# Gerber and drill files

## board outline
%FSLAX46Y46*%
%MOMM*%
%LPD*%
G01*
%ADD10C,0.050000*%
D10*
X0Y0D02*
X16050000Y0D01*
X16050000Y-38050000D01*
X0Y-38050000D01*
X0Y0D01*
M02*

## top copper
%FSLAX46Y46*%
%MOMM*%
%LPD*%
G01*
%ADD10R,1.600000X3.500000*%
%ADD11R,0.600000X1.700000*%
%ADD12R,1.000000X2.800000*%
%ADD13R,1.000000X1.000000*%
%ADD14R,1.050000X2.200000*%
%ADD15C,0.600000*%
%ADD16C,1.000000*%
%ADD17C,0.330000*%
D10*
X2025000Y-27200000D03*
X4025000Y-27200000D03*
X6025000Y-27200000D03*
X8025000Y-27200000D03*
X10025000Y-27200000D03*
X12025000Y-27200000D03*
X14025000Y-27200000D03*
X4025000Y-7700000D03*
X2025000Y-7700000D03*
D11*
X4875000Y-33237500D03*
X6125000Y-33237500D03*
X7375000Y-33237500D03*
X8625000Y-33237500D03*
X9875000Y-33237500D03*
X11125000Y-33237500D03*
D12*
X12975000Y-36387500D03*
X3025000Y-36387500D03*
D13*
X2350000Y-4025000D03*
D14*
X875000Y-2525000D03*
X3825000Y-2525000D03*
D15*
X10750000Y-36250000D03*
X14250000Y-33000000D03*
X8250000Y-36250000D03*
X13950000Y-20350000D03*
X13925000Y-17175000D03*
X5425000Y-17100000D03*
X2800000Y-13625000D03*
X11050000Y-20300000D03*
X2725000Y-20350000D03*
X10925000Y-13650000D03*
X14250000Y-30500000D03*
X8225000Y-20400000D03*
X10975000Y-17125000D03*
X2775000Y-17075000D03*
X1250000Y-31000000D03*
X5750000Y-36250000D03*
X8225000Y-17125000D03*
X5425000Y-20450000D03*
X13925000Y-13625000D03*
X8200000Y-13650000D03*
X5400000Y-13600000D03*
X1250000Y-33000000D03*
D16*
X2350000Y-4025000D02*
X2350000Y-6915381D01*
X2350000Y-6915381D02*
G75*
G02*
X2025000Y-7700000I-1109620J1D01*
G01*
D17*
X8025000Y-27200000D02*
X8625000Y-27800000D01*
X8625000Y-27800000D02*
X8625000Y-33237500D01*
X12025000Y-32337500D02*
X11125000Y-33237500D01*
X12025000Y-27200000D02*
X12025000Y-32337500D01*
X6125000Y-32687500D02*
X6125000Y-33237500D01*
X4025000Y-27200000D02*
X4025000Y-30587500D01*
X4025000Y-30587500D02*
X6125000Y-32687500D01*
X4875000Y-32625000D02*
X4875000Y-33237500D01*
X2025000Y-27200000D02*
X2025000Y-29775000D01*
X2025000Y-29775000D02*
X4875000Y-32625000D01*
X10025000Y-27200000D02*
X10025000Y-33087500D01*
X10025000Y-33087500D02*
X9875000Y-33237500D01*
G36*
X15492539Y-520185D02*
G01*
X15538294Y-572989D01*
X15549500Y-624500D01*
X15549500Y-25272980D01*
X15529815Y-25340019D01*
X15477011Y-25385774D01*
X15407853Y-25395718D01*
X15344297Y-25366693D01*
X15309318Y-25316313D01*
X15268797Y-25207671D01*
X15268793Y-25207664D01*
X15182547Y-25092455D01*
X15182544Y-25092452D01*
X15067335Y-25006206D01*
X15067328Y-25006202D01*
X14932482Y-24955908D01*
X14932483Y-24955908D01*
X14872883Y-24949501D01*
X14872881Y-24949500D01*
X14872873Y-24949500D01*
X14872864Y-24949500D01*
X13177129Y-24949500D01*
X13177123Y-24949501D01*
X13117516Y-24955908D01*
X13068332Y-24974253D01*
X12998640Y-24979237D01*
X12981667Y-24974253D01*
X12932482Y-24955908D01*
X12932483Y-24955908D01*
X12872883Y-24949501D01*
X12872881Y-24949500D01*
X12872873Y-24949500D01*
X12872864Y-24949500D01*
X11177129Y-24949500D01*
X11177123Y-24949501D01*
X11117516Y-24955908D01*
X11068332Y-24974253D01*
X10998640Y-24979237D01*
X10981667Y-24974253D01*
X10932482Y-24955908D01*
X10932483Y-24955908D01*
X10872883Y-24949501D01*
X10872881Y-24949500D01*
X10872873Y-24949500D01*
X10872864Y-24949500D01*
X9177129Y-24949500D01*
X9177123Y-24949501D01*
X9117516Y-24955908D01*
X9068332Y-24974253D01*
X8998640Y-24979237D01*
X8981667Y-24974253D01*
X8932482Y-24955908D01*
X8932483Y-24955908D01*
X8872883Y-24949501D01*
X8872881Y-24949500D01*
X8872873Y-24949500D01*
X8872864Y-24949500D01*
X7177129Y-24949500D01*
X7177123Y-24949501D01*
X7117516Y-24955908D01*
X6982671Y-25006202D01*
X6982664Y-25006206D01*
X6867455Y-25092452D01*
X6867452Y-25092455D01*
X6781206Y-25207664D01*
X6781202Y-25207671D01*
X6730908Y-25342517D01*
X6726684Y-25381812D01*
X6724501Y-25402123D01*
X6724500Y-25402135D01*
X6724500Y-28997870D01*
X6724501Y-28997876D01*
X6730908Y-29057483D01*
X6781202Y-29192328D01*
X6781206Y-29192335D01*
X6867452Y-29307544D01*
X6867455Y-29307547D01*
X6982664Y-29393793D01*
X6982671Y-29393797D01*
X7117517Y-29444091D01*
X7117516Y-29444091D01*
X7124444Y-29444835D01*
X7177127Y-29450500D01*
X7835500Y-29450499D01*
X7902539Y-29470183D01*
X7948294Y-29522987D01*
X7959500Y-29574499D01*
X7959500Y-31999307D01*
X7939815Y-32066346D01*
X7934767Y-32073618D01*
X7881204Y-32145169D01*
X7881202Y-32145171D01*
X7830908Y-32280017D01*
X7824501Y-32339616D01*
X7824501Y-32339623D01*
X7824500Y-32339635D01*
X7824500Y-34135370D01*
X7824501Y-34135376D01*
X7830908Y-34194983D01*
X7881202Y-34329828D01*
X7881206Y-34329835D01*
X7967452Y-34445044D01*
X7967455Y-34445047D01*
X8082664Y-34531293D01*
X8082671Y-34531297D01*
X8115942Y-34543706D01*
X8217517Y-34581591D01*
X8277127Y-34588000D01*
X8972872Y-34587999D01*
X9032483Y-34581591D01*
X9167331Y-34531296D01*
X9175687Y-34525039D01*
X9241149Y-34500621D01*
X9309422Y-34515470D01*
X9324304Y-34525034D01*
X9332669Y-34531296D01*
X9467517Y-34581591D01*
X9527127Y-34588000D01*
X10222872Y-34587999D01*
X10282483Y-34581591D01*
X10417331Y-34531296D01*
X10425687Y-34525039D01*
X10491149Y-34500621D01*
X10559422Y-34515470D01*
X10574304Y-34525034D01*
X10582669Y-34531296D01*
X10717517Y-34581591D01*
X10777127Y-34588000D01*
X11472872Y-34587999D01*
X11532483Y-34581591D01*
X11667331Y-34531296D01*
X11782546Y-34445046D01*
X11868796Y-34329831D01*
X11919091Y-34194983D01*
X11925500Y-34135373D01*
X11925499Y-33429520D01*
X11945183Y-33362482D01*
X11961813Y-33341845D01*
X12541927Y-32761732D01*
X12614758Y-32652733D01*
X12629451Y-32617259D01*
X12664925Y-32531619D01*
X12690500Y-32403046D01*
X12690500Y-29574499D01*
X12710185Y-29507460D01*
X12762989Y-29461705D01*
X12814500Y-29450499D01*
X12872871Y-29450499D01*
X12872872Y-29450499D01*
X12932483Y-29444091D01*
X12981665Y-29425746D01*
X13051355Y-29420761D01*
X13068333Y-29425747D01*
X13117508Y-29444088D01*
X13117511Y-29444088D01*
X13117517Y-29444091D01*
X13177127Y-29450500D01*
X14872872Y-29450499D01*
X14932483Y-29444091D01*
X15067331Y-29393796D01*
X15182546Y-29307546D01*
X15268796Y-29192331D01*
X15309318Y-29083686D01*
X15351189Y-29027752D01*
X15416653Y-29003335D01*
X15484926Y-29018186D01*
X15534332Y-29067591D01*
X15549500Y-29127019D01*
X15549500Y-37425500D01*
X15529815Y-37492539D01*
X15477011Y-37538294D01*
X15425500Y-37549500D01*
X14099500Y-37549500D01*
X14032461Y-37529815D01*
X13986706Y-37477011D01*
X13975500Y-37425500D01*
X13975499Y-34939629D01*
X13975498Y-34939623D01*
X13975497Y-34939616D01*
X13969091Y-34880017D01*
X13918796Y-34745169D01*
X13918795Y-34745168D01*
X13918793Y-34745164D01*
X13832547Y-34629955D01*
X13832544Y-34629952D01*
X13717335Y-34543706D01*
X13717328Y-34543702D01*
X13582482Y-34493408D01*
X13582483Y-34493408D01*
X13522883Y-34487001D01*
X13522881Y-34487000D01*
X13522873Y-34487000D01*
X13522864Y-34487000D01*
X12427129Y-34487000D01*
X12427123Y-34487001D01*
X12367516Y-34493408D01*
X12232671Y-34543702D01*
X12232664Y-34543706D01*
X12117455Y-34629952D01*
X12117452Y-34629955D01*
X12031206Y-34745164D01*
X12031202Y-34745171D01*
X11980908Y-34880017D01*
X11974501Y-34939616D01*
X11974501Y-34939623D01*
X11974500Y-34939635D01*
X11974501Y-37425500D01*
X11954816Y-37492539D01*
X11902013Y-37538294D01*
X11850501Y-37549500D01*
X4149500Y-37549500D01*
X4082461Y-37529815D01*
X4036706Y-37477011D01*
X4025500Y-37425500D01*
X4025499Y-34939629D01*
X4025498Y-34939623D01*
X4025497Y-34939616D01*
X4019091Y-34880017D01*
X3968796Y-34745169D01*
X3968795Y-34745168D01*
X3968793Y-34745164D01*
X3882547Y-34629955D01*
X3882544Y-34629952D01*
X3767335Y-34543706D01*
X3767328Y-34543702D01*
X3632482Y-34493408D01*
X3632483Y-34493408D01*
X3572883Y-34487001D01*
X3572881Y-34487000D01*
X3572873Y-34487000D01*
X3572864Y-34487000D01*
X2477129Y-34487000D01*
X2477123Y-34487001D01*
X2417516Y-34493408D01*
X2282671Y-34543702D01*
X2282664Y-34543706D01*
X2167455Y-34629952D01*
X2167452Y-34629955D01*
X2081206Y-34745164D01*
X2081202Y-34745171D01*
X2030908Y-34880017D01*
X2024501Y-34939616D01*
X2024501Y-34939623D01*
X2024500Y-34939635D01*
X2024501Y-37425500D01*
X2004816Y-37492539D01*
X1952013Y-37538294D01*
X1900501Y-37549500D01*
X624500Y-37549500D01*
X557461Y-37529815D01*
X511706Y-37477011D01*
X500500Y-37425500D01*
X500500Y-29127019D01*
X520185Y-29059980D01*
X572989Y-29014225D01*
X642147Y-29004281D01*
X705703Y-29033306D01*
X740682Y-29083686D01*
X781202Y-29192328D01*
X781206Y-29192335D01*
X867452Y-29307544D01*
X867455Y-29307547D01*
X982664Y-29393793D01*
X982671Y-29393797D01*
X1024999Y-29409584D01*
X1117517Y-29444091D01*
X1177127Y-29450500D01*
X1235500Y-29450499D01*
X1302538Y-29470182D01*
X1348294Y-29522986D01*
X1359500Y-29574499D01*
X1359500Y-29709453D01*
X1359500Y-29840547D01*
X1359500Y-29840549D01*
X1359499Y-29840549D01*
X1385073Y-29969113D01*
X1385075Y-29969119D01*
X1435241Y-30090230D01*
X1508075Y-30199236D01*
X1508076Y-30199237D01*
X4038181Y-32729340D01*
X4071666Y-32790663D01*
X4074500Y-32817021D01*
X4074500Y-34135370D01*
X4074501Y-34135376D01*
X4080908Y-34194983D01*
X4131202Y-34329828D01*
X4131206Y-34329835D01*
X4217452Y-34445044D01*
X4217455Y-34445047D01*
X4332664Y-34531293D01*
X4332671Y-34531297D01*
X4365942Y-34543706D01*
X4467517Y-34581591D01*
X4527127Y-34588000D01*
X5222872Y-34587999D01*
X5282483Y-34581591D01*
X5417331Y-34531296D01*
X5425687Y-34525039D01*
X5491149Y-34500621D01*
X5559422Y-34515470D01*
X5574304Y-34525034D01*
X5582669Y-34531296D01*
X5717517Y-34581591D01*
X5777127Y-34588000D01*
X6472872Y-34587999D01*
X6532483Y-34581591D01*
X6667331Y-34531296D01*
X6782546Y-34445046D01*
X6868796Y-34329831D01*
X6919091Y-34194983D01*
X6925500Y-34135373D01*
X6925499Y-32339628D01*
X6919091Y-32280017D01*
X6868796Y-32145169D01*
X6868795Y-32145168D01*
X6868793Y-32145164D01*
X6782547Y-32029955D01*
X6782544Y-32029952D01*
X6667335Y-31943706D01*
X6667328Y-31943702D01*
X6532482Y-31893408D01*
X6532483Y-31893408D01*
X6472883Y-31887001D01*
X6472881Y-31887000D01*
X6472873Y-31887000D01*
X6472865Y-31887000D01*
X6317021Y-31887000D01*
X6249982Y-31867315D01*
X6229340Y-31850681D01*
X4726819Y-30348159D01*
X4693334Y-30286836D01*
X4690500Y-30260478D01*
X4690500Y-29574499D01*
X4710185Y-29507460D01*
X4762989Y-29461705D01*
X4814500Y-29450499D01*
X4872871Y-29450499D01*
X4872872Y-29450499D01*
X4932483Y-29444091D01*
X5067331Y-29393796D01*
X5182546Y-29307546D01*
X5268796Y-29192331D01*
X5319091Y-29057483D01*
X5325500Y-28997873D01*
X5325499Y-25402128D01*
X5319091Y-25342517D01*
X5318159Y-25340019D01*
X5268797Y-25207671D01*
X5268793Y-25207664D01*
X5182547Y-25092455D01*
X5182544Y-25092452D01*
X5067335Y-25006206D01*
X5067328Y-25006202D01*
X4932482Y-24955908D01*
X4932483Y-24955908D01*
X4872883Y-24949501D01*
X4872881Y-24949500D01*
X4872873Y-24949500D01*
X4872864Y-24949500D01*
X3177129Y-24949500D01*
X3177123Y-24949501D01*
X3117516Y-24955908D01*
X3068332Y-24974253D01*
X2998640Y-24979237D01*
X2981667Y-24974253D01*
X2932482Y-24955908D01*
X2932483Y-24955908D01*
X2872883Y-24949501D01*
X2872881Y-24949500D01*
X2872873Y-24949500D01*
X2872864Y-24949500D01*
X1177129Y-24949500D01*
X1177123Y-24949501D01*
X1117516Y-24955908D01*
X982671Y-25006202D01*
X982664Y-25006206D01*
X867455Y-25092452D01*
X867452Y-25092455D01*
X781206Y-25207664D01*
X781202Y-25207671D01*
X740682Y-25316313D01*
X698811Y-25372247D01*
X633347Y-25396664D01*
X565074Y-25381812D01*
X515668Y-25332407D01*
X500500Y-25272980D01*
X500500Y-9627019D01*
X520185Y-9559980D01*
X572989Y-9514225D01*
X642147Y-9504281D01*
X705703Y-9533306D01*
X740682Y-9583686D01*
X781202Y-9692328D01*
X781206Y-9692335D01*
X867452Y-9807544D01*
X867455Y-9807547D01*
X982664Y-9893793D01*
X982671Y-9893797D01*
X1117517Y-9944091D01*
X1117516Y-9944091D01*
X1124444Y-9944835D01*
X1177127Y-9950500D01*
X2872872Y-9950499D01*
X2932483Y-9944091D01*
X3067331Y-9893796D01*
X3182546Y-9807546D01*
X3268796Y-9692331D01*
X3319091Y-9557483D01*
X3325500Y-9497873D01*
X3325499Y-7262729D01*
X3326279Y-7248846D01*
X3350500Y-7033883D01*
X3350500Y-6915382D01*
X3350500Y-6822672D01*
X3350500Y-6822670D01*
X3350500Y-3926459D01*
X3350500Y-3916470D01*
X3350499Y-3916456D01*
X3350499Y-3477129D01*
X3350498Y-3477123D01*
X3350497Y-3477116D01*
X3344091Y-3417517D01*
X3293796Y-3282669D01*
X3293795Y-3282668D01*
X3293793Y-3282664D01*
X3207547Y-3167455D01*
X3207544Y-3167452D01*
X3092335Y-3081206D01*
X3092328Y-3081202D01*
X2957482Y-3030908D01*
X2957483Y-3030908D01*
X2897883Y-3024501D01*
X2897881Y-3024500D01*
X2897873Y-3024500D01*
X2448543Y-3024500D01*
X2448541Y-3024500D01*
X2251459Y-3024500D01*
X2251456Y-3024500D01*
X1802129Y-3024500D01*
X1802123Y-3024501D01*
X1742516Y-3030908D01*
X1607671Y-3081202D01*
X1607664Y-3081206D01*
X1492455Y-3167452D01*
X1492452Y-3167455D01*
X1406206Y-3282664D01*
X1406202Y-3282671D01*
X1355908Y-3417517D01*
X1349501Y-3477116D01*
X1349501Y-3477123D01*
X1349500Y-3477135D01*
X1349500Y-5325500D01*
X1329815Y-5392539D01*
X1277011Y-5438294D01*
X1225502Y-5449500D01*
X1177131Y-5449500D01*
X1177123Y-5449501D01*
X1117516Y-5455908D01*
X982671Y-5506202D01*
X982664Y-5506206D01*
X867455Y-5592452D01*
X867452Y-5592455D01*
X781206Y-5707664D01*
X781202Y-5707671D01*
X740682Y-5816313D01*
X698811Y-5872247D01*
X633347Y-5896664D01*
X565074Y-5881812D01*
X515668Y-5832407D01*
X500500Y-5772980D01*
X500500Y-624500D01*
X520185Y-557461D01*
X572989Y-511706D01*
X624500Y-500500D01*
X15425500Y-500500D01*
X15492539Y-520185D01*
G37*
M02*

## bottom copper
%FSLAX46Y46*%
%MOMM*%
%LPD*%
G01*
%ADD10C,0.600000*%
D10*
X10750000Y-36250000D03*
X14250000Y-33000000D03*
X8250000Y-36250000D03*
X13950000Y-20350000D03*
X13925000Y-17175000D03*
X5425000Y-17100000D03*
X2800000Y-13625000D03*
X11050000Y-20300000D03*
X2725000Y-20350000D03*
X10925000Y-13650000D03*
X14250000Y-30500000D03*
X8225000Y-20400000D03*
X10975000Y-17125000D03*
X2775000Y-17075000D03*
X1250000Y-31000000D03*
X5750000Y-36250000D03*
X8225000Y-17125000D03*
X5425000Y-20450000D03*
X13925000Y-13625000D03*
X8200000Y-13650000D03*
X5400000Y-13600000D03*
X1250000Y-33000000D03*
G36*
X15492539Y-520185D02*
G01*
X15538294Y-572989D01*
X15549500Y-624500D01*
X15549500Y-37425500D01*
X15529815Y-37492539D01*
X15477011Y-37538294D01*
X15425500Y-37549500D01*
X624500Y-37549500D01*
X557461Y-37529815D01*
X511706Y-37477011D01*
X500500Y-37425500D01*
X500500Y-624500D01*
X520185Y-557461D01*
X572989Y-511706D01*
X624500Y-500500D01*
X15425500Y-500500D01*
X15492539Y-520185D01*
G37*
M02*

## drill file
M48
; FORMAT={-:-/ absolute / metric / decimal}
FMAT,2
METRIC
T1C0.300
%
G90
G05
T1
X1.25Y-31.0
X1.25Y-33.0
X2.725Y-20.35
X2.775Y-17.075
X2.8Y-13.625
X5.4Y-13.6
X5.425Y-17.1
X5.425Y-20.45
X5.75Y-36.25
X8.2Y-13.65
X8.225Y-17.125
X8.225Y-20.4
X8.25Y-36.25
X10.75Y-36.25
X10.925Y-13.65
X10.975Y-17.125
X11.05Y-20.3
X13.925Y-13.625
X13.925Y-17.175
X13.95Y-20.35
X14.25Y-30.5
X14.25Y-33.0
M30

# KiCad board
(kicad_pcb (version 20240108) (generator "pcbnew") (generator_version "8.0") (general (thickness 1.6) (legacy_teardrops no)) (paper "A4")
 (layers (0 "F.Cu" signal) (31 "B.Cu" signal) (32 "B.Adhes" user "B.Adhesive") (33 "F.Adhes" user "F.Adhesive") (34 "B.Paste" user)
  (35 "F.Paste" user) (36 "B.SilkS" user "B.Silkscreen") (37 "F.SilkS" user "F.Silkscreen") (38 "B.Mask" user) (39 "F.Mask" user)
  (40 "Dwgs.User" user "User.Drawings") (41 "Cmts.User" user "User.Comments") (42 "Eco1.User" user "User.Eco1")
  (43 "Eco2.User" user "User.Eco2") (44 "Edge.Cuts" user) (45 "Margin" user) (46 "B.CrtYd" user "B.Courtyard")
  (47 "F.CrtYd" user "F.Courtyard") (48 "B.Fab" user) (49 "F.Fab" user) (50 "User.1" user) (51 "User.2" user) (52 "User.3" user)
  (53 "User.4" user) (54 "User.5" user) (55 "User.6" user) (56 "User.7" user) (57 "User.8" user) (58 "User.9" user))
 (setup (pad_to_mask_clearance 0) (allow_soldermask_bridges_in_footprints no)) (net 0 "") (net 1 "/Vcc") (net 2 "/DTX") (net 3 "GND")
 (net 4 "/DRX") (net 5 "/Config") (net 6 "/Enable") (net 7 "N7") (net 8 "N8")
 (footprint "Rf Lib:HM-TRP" (layer "F.Cu") (at 0.025 27.45)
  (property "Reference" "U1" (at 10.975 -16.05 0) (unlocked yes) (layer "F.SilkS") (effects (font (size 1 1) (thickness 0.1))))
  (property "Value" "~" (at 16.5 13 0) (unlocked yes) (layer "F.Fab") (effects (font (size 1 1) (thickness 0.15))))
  (pad "1" smd rect (at 2 -0.25 180) (size 1.6 3.5) (layers "F.Cu" "F.Paste" "F.Mask") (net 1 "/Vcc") (thermal_bridge_angle 45))
  (pad "2" smd rect (at 4 -0.25 180) (size 1.6 3.5) (layers "F.Cu" "F.Paste" "F.Mask") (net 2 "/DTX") (thermal_bridge_angle 45))
  (pad "3" smd rect (at 6 -0.25 180) (size 1.6 3.5) (layers "F.Cu" "F.Paste" "F.Mask") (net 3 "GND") (zone_connect 2)
   (thermal_bridge_angle 45))
  (pad "4" smd rect (at 8 -0.25 180) (size 1.6 3.5) (layers "F.Cu" "F.Paste" "F.Mask") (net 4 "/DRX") (thermal_bridge_angle 45))
  (pad "5" smd rect (at 10 -0.25 180) (size 1.6 3.5) (layers "F.Cu" "F.Paste" "F.Mask") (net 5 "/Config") (thermal_bridge_angle 45))
  (pad "6" smd rect (at 12 -0.25 180) (size 1.6 3.5) (layers "F.Cu" "F.Paste" "F.Mask") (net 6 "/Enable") (thermal_bridge_angle 45))
  (pad "7" smd rect (at 14 -0.25 180) (size 1.6 3.5) (layers "F.Cu" "F.Paste" "F.Mask") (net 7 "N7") (thermal_bridge_angle 45))
  (pad "8" smd rect (at 4 -19.75 180) (size 1.6 3.5) (layers "F.Cu" "F.Paste" "F.Mask") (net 3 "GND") (zone_connect 2)
   (thermal_bridge_angle 45))
  (pad "9" smd rect (at 2 -19.75 180) (size 1.6 3.5) (layers "F.Cu" "F.Paste" "F.Mask") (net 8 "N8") (thermal_bridge_angle 45)))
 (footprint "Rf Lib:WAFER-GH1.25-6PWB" (layer "F.Cu") (at 8 34.8125)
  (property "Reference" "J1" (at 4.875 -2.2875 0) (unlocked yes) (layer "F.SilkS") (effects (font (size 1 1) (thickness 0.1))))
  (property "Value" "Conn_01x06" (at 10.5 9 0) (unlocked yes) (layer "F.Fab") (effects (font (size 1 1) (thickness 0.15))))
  (pad "1" smd rect (at -3.125 -1.575 180) (size 0.6 1.7) (layers "F.Cu" "F.Paste" "F.Mask") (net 1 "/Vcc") (thermal_bridge_angle 45))
  (pad "2" smd rect (at -1.875 -1.575 180) (size 0.6 1.7) (layers "F.Cu" "F.Paste" "F.Mask") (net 2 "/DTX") (thermal_bridge_angle 45))
  (pad "3" smd rect (at -0.625 -1.575 180) (size 0.6 1.7) (layers "F.Cu" "F.Paste" "F.Mask") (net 3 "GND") (zone_connect 2)
   (thermal_bridge_angle 45))
  (pad "4" smd rect (at 0.625 -1.575 180) (size 0.6 1.7) (layers "F.Cu" "F.Paste" "F.Mask") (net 4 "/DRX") (thermal_bridge_angle 45))
  (pad "5" smd rect (at 1.875 -1.575 180) (size 0.6 1.7) (layers "F.Cu" "F.Paste" "F.Mask") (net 5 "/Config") (thermal_bridge_angle 45))
  (pad "6" smd rect (at 3.125 -1.575 180) (size 0.6 1.7) (layers "F.Cu" "F.Paste" "F.Mask") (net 6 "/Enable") (thermal_bridge_angle 45))
  (pad "7" smd rect (at 4.975 1.575 180) (size 1 2.8) (layers "F.Cu" "F.Paste" "F.Mask") (thermal_bridge_angle 45))
  (pad "8" smd rect (at -4.975 1.575 180) (size 1 2.8) (layers "F.Cu" "F.Paste" "F.Mask") (thermal_bridge_angle 45)))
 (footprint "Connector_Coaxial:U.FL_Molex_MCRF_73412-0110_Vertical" (layer "F.Cu") (at 2.35 2.525)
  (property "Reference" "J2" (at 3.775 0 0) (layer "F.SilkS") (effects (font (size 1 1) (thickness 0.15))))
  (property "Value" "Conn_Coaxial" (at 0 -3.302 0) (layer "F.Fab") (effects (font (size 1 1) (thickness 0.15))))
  (pad "1" smd rect (at 0 1.5) (size 1 1) (layers "F.Cu" "F.Paste" "F.Mask") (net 8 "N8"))
  (pad "2" smd rect (at -1.475 0) (size 1.05 2.2) (layers "F.Cu" "F.Paste" "F.Mask") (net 3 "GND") (zone_connect 2))
  (pad "2" smd rect (at 1.475 0) (size 1.05 2.2) (layers "F.Cu" "F.Paste" "F.Mask") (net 3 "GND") (zone_connect 2)))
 (gr_rect (start 0 0) (end 16.05 38.05) (stroke (width 0.05) (type default)) (fill none) (layer "Edge.Cuts"))
 (via (at 10.75 36.25) (size 0.6) (drill 0.3) (layers "F.Cu" "B.Cu") (free yes) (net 3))
 (via (at 14.25 33) (size 0.6) (drill 0.3) (layers "F.Cu" "B.Cu") (free yes) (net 3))
 (via (at 8.25 36.25) (size 0.6) (drill 0.3) (layers "F.Cu" "B.Cu") (free yes) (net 3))
 (via (at 13.95 20.35) (size 0.6) (drill 0.3) (layers "F.Cu" "B.Cu") (free yes) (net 3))
 (via (at 13.925 17.175) (size 0.6) (drill 0.3) (layers "F.Cu" "B.Cu") (free yes) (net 3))
 (via (at 5.425 17.1) (size 0.6) (drill 0.3) (layers "F.Cu" "B.Cu") (free yes) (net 3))
 (via (at 2.8 13.625) (size 0.6) (drill 0.3) (layers "F.Cu" "B.Cu") (free yes) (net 3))
 (via (at 11.05 20.3) (size 0.6) (drill 0.3) (layers "F.Cu" "B.Cu") (free yes) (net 3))
 (via (at 2.725 20.35) (size 0.6) (drill 0.3) (layers "F.Cu" "B.Cu") (free yes) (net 3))
 (via (at 10.925 13.65) (size 0.6) (drill 0.3) (layers "F.Cu" "B.Cu") (free yes) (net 3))
 (via (at 14.25 30.5) (size 0.6) (drill 0.3) (layers "F.Cu" "B.Cu") (free yes) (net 3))
 (via (at 8.225 20.4) (size 0.6) (drill 0.3) (layers "F.Cu" "B.Cu") (free yes) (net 3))
 (via (at 10.975 17.125) (size 0.6) (drill 0.3) (layers "F.Cu" "B.Cu") (free yes) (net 3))
 (via (at 2.775 17.075) (size 0.6) (drill 0.3) (layers "F.Cu" "B.Cu") (free yes) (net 3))
 (via (at 1.25 31) (size 0.6) (drill 0.3) (layers "F.Cu" "B.Cu") (free yes) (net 3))
 (via (at 5.75 36.25) (size 0.6) (drill 0.3) (layers "F.Cu" "B.Cu") (free yes) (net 3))
 (via (at 8.225 17.125) (size 0.6) (drill 0.3) (layers "F.Cu" "B.Cu") (free yes) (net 3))
 (via (at 5.425 20.45) (size 0.6) (drill 0.3) (layers "F.Cu" "B.Cu") (free yes) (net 3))
 (via (at 13.925 13.625) (size 0.6) (drill 0.3) (layers "F.Cu" "B.Cu") (free yes) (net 3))
 (via (at 8.2 13.65) (size 0.6) (drill 0.3) (layers "F.Cu" "B.Cu") (free yes) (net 3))
 (via (at 5.4 13.6) (size 0.6) (drill 0.3) (layers "F.Cu" "B.Cu") (free yes) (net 3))
 (via (at 1.25 33) (size 0.6) (drill 0.3) (layers "F.Cu" "B.Cu") (free yes) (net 3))
 (segment (start 2.35 4.025) (end 2.35 6.915381) (width 1) (layer "F.Cu") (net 8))
 (arc (start 2.35 6.915381) (mid 2.265535 7.340014) (end 2.025 7.7) (width 1) (layer "F.Cu") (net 8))
 (segment (start 8.025 27.2) (end 8.625 27.8) (width 0.33) (layer "F.Cu") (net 4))
 (segment (start 8.625 27.8) (end 8.625 33.2375) (width 0.33) (layer "F.Cu") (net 4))
 (segment (start 12.025 32.3375) (end 11.125 33.2375) (width 0.33) (layer "F.Cu") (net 6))
 (segment (start 12.025 27.2) (end 12.025 32.3375) (width 0.33) (layer "F.Cu") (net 6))
 (segment (start 6.125 32.6875) (end 6.125 33.2375) (width 0.33) (layer "F.Cu") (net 2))
 (segment (start 4.025 27.2) (end 4.025 30.5875) (width 0.33) (layer "F.Cu") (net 2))
 (segment (start 4.025 30.5875) (end 6.125 32.6875) (width 0.33) (layer "F.Cu") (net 2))
 (segment (start 4.875 32.625) (end 4.875 33.2375) (width 0.33) (layer "F.Cu") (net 1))
 (segment (start 2.025 27.2) (end 2.025 29.775) (width 0.33) (layer "F.Cu") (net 1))
 (segment (start 2.025 29.775) (end 4.875 32.625) (width 0.33) (layer "F.Cu") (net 1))
 (segment (start 10.025 27.2) (end 10.025 33.0875) (width 0.33) (layer "F.Cu") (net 5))
 (segment (start 10.025 33.0875) (end 9.875 33.2375) (width 0.33) (layer "F.Cu") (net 5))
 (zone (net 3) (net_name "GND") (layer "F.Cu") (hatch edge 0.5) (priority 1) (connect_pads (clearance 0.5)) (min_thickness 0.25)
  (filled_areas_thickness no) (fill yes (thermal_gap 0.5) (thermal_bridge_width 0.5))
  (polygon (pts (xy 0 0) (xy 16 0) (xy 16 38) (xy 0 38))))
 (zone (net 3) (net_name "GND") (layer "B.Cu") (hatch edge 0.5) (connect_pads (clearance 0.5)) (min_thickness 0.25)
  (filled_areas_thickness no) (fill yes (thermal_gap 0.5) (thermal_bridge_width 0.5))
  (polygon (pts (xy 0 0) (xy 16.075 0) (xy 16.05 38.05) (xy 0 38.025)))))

